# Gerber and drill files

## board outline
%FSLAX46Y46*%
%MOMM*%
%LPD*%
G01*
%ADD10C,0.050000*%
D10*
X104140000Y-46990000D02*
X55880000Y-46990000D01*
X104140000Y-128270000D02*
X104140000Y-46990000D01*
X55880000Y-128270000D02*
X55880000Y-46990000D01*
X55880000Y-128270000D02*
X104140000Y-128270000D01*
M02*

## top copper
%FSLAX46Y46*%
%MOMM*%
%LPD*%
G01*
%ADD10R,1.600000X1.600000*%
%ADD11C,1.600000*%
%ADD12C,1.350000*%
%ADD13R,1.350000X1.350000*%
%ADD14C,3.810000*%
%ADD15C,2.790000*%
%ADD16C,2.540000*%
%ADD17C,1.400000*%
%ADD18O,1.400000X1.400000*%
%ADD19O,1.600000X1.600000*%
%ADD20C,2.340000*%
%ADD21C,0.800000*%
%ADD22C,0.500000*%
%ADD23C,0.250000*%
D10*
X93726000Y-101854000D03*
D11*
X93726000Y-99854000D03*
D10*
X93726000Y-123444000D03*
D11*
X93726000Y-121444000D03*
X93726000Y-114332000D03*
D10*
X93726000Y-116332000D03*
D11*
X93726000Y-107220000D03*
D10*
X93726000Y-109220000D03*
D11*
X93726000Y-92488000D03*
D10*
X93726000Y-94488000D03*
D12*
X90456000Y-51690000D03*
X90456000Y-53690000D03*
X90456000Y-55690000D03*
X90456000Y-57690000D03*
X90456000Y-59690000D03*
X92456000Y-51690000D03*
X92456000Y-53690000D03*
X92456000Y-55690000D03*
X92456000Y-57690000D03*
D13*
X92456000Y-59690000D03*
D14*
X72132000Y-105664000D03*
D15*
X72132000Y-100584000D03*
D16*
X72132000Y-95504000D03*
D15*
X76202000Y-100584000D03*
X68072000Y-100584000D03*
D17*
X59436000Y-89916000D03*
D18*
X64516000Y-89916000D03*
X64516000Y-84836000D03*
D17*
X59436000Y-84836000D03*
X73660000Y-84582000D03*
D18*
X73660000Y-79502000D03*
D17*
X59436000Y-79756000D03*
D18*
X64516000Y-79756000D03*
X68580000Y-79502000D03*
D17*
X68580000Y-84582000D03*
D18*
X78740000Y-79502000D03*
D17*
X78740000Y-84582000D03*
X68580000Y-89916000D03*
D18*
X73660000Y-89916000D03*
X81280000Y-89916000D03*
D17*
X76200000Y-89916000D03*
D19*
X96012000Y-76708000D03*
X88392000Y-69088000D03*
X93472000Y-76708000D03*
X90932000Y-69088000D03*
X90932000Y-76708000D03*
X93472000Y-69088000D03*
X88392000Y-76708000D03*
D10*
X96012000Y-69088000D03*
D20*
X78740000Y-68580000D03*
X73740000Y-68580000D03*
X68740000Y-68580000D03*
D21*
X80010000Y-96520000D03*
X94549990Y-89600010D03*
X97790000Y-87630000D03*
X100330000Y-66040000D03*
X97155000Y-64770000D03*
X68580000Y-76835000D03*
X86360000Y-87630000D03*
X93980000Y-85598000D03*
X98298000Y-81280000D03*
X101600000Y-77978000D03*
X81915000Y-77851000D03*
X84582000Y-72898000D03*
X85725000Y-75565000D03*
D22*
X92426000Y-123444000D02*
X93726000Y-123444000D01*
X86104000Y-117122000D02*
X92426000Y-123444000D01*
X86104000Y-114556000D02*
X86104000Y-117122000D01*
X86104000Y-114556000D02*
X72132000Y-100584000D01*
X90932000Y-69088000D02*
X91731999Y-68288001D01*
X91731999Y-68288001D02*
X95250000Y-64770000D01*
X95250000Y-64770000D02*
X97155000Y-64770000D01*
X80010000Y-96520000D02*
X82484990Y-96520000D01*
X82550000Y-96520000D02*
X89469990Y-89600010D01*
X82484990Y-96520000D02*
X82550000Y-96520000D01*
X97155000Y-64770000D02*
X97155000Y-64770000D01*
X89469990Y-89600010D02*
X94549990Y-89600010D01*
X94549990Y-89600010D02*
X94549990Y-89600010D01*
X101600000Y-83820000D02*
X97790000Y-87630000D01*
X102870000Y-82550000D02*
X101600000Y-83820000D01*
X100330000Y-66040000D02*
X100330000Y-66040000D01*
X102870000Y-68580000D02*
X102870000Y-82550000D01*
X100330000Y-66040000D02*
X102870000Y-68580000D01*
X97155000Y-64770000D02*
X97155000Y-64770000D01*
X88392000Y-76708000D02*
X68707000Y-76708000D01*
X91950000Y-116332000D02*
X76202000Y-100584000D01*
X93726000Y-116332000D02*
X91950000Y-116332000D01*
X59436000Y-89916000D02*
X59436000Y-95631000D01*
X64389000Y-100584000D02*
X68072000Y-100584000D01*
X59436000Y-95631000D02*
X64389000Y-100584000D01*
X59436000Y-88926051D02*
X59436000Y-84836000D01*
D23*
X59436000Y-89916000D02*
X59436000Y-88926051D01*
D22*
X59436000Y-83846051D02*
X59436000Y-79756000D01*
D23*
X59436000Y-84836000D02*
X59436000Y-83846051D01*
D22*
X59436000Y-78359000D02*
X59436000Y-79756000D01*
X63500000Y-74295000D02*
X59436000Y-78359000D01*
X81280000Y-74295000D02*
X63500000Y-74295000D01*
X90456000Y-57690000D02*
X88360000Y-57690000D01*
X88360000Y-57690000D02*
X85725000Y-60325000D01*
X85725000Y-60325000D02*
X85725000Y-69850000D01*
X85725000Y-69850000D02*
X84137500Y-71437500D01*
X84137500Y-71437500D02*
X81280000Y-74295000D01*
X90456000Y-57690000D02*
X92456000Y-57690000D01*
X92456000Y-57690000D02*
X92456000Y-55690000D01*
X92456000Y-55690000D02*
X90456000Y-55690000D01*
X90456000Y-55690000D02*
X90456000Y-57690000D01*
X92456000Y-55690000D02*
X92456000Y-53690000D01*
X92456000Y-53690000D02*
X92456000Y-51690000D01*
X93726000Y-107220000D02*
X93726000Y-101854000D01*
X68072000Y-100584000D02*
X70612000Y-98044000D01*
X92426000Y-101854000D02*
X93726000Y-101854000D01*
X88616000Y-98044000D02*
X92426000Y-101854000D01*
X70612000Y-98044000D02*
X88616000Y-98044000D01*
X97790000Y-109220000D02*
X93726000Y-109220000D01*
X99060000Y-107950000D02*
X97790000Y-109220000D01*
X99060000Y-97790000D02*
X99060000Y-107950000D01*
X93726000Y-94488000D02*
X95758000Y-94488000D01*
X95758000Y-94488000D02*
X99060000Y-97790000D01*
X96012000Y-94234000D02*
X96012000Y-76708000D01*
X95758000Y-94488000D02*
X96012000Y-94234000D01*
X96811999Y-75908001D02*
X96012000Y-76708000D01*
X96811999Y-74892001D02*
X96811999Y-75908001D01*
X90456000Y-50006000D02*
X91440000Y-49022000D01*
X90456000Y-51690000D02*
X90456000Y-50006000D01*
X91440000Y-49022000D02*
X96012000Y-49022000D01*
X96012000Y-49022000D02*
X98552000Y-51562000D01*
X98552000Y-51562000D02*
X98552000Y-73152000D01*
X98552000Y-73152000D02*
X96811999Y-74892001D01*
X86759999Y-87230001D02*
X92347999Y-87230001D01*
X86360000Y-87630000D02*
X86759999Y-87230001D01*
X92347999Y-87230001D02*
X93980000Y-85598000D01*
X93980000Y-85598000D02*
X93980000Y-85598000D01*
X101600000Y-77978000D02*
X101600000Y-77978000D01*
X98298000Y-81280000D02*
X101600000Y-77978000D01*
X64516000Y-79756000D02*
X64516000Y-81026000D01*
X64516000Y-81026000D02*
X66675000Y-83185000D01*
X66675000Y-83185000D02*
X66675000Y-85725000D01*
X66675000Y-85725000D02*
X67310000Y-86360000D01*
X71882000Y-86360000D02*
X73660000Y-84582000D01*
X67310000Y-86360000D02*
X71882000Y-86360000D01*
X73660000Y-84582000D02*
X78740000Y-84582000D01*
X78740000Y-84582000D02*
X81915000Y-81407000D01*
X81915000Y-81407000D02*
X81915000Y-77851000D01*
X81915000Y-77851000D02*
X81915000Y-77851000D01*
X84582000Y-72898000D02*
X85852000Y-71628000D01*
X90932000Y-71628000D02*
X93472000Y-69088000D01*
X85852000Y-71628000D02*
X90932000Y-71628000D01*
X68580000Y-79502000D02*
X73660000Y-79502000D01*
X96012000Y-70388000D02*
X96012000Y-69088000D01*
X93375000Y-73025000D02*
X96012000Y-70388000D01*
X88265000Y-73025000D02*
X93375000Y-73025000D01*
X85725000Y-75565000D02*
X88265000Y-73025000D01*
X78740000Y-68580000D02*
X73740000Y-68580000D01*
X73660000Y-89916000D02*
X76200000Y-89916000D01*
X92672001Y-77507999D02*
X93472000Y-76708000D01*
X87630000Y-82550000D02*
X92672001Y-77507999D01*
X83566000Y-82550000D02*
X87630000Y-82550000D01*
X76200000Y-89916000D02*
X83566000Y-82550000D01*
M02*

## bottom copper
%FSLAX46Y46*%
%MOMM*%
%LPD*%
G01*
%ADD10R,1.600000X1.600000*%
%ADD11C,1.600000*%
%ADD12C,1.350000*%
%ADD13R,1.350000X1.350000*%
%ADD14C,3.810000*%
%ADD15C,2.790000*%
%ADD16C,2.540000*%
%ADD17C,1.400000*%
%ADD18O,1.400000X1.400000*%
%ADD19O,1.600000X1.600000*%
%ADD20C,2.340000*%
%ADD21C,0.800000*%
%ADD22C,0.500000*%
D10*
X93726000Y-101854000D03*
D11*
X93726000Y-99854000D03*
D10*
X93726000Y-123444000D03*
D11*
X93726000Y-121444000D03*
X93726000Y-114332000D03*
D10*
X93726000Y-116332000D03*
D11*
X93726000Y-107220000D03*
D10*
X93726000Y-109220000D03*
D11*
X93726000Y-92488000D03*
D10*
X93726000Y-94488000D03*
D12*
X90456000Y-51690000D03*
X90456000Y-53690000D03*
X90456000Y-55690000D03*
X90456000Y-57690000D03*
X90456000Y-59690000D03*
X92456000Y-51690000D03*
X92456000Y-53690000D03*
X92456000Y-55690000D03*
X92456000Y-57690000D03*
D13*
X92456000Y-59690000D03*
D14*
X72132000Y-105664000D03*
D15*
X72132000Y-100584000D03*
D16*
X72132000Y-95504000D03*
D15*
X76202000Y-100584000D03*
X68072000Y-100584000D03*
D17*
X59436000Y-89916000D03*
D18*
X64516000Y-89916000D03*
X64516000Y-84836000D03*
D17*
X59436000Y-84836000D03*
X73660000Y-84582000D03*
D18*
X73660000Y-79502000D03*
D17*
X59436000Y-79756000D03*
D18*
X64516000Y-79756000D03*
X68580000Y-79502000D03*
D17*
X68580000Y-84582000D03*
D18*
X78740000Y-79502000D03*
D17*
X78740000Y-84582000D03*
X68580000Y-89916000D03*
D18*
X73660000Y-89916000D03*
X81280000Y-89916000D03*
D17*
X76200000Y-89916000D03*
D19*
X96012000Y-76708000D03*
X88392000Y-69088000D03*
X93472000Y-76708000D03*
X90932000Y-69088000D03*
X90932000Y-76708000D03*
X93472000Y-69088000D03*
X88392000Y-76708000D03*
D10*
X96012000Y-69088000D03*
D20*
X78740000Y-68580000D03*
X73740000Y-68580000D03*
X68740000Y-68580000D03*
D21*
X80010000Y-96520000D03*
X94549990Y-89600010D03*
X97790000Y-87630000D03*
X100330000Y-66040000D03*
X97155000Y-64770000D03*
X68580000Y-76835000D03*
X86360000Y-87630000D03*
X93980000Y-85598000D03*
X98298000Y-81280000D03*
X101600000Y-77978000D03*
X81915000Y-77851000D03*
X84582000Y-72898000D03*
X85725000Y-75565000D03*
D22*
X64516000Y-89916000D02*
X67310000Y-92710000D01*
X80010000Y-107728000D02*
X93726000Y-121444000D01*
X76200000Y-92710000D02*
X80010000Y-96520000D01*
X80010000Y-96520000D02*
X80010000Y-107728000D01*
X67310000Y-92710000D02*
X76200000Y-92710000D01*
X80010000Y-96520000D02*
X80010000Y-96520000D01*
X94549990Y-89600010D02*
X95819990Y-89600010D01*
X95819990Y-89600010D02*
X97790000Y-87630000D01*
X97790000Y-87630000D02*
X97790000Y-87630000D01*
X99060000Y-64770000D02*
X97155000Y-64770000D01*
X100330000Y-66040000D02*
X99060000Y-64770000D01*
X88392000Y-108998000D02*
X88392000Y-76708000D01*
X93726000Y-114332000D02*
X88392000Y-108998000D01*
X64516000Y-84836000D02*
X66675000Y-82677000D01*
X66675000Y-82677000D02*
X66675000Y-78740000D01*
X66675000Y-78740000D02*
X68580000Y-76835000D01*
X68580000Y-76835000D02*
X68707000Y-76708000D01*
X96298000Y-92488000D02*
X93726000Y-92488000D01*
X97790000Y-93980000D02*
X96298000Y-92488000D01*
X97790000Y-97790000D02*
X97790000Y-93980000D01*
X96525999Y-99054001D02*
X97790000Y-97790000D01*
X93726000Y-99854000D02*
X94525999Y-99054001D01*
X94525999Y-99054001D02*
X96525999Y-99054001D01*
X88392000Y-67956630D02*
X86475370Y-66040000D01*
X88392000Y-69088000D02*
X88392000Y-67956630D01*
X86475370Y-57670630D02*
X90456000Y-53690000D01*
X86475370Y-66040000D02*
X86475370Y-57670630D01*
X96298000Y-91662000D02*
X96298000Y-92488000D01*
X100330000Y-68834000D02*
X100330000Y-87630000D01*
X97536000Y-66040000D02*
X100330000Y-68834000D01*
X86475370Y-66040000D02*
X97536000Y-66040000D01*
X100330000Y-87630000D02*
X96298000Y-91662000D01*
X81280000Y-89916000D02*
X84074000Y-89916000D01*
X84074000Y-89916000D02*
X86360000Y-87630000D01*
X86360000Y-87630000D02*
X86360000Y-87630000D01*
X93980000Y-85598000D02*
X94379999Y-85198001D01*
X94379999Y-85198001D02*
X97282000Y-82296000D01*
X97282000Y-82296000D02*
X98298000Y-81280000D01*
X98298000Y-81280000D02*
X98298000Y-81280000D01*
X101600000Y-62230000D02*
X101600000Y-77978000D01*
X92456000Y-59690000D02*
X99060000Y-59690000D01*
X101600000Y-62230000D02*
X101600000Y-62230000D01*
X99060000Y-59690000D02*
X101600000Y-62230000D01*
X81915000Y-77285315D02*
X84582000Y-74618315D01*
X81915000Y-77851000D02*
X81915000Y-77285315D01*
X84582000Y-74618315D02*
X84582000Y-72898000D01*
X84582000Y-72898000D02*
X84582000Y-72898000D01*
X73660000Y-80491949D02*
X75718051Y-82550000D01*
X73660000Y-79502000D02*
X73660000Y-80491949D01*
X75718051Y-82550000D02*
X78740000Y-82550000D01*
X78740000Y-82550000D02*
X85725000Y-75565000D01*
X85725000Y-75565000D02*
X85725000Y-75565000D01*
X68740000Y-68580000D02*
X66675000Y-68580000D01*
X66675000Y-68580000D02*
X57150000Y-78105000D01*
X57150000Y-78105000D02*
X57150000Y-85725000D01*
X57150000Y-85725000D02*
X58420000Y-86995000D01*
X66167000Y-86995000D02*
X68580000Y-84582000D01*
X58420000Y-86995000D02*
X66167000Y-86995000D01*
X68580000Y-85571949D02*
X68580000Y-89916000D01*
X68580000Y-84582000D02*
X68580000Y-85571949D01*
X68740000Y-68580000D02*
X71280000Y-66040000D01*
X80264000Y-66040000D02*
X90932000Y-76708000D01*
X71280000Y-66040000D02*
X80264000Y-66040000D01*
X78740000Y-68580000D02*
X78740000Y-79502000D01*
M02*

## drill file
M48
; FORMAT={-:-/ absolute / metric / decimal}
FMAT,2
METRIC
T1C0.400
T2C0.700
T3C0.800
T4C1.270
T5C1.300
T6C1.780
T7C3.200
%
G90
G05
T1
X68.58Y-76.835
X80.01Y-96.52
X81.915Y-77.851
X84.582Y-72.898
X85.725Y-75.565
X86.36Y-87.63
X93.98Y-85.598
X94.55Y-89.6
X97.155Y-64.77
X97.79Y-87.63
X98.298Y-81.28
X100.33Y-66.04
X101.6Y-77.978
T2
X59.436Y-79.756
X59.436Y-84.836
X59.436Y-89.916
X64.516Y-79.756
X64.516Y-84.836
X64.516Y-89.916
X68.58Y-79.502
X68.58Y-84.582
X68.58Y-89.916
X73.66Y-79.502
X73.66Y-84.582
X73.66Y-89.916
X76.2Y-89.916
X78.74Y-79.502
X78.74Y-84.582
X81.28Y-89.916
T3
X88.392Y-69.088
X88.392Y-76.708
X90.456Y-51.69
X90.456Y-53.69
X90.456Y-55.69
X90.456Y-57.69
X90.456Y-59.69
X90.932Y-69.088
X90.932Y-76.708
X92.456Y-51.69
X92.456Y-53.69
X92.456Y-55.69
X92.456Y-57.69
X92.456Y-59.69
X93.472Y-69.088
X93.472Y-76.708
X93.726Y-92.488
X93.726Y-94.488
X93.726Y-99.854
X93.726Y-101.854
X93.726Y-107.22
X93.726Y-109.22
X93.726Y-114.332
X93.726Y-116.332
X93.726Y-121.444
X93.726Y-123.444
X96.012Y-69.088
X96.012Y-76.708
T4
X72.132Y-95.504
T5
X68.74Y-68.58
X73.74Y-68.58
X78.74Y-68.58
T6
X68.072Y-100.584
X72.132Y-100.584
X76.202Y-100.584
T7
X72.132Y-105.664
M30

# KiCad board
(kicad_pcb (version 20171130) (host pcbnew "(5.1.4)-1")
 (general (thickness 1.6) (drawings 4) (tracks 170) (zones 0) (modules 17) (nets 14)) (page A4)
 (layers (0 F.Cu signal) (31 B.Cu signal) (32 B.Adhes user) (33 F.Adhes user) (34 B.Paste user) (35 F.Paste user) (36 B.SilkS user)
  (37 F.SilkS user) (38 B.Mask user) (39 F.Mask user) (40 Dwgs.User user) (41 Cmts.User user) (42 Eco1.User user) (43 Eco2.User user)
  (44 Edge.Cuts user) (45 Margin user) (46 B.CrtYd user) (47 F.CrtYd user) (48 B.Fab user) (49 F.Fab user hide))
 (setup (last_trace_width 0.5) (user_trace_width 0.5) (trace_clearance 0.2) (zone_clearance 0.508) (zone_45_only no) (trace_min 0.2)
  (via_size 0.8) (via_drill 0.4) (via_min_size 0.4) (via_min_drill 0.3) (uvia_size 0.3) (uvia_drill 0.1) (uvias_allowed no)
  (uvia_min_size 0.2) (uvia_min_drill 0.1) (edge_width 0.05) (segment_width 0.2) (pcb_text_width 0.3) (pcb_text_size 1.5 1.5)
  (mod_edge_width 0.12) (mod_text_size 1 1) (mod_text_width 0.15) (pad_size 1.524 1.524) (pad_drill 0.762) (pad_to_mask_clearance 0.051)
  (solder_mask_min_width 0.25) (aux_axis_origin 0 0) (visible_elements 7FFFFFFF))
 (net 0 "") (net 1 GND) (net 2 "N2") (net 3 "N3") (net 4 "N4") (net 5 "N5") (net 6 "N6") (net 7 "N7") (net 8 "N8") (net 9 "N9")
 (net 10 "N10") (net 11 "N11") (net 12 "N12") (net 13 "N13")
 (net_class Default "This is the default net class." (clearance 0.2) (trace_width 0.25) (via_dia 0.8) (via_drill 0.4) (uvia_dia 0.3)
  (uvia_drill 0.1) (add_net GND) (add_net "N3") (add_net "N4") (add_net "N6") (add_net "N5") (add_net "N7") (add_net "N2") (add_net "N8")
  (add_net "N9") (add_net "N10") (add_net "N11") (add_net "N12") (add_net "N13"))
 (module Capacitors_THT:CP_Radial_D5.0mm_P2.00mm (layer F.Cu) (at 93.726 101.854 90)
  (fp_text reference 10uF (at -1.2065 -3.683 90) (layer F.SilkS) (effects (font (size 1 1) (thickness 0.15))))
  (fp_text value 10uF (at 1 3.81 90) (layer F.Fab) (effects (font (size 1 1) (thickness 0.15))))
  (pad 1 thru_hole rect (at 0 0 90) (size 1.6 1.6) (drill 0.8) (layers *.Cu *.Mask) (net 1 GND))
  (pad 2 thru_hole circle (at 2 0 90) (size 1.6 1.6) (drill 0.8) (layers *.Cu *.Mask) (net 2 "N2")))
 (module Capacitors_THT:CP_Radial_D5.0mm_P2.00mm (layer F.Cu) (at 93.726 123.444 90)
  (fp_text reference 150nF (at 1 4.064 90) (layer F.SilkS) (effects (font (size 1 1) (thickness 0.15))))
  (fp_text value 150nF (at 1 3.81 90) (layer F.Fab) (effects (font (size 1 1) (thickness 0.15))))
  (pad 1 thru_hole rect (at 0 0 90) (size 1.6 1.6) (drill 0.8) (layers *.Cu *.Mask) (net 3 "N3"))
  (pad 2 thru_hole circle (at 2 0 90) (size 1.6 1.6) (drill 0.8) (layers *.Cu *.Mask) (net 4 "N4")))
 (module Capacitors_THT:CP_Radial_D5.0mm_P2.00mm (layer F.Cu) (at 93.726 116.332 90)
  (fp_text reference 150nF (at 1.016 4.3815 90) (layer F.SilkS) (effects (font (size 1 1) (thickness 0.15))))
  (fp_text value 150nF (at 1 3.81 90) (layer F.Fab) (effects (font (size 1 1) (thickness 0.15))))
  (pad 2 thru_hole circle (at 2 0 90) (size 1.6 1.6) (drill 0.8) (layers *.Cu *.Mask) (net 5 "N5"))
  (pad 1 thru_hole rect (at 0 0 90) (size 1.6 1.6) (drill 0.8) (layers *.Cu *.Mask) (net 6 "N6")))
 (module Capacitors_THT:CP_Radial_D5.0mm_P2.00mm (layer F.Cu) (at 93.726 109.22 90)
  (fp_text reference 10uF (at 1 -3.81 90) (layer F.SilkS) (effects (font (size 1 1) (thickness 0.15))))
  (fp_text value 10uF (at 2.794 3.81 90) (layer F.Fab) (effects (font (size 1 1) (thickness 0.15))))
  (pad 2 thru_hole circle (at 2 0 90) (size 1.6 1.6) (drill 0.8) (layers *.Cu *.Mask) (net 1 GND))
  (pad 1 thru_hole rect (at 0 0 90) (size 1.6 1.6) (drill 0.8) (layers *.Cu *.Mask) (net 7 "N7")))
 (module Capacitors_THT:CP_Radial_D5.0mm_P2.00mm (layer F.Cu) (at 93.726 94.488 90)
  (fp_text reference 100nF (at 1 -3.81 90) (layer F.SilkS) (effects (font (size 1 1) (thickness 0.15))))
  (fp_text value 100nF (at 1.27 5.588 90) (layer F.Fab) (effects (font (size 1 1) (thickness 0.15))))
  (pad 2 thru_hole circle (at 2 0 90) (size 1.6 1.6) (drill 0.8) (layers *.Cu *.Mask) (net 2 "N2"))
  (pad 1 thru_hole rect (at 0 0 90) (size 1.6 1.6) (drill 0.8) (layers *.Cu *.Mask) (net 7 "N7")))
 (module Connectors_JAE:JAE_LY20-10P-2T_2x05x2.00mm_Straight (layer F.Cu) (at 92.456 59.69 90)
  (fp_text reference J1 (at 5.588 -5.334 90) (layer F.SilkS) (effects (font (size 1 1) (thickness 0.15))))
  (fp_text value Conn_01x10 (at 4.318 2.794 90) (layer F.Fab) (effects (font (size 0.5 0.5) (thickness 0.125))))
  (pad 10 thru_hole circle (at 8 -2 90) (size 1.35 1.35) (drill 0.8) (layers *.Cu *.Mask) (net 7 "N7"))
  (pad 9 thru_hole circle (at 6 -2 90) (size 1.35 1.35) (drill 0.8) (layers *.Cu *.Mask) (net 2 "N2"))
  (pad 8 thru_hole circle (at 4 -2 90) (size 1.35 1.35) (drill 0.8) (layers *.Cu *.Mask) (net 1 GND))
  (pad 7 thru_hole circle (at 2 -2 90) (size 1.35 1.35) (drill 0.8) (layers *.Cu *.Mask) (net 1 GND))
  (pad 6 thru_hole circle (at 0 -2 90) (size 1.35 1.35) (drill 0.8) (layers *.Cu *.Mask))
  (pad 5 thru_hole circle (at 8 0 90) (size 1.35 1.35) (drill 0.8) (layers *.Cu *.Mask) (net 1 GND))
  (pad 4 thru_hole circle (at 6 0 90) (size 1.35 1.35) (drill 0.8) (layers *.Cu *.Mask) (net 1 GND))
  (pad 3 thru_hole circle (at 4 0 90) (size 1.35 1.35) (drill 0.8) (layers *.Cu *.Mask) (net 1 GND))
  (pad 2 thru_hole circle (at 2 0 90) (size 1.35 1.35) (drill 0.8) (layers *.Cu *.Mask) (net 1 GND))
  (pad 1 thru_hole rect (at 0 0 90) (size 1.35 1.35) (drill 0.8) (layers *.Cu *.Mask) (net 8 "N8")))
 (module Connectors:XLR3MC (layer F.Cu) (at 68.072 100.584)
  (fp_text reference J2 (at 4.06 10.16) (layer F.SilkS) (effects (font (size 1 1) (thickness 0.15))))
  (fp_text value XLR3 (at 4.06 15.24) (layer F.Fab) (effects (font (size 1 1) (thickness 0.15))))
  (pad "" thru_hole circle (at 4.06 5.08) (size 3.81 3.81) (drill 3.2) (layers *.Cu *.Mask))
  (pad 3 thru_hole circle (at 4.06 0) (size 2.79 2.79) (drill 1.78) (layers *.Cu *.Mask) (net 3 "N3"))
  (pad 4 thru_hole circle (at 4.06 -5.08) (size 2.54 2.54) (drill 1.27) (layers *.Cu *.Mask))
  (pad 2 thru_hole circle (at 8.13 0) (size 2.79 2.79) (drill 1.78) (layers *.Cu *.Mask) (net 6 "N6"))
  (pad 1 thru_hole circle (at 0 0) (size 2.79 2.79) (drill 1.78) (layers *.Cu *.Mask) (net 1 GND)))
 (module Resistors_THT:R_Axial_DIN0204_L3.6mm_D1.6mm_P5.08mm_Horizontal (layer F.Cu) (at 59.436 89.916)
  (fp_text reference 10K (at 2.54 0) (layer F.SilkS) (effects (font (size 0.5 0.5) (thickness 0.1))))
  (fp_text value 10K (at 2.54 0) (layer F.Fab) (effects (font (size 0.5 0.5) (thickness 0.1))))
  (pad 1 thru_hole circle (at 0 0) (size 1.4 1.4) (drill 0.7) (layers *.Cu *.Mask) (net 1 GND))
  (pad 2 thru_hole oval (at 5.08 0) (size 1.4 1.4) (drill 0.7) (layers *.Cu *.Mask) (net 4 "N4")))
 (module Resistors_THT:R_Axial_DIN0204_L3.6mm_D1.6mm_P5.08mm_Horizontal (layer F.Cu) (at 59.436 84.836)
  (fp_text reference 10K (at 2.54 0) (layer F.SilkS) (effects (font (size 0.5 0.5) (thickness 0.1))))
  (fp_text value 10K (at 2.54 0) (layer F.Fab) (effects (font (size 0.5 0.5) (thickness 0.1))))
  (pad 2 thru_hole oval (at 5.08 0) (size 1.4 1.4) (drill 0.7) (layers *.Cu *.Mask) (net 5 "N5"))
  (pad 1 thru_hole circle (at 0 0) (size 1.4 1.4) (drill 0.7) (layers *.Cu *.Mask) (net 1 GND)))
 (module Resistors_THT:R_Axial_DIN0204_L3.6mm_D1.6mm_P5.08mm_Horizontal (layer F.Cu) (at 73.66 84.582 90)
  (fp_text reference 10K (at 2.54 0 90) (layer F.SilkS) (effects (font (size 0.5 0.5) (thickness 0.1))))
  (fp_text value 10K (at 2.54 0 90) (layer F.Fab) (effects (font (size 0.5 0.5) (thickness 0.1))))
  (pad 1 thru_hole circle (at 0 0 90) (size 1.4 1.4) (drill 0.7) (layers *.Cu *.Mask) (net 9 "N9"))
  (pad 2 thru_hole oval (at 5.08 0 90) (size 1.4 1.4) (drill 0.7) (layers *.Cu *.Mask) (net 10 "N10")))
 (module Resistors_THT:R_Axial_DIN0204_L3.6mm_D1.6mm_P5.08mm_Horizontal (layer F.Cu) (at 59.436 79.756)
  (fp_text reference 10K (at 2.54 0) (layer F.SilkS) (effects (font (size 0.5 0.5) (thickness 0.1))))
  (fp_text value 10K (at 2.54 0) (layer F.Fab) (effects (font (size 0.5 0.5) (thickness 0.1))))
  (pad 1 thru_hole circle (at 0 0) (size 1.4 1.4) (drill 0.7) (layers *.Cu *.Mask) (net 1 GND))
  (pad 2 thru_hole oval (at 5.08 0) (size 1.4 1.4) (drill 0.7) (layers *.Cu *.Mask) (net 9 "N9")))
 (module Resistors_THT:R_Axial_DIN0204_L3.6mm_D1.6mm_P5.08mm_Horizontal (layer F.Cu) (at 68.58 84.582 90)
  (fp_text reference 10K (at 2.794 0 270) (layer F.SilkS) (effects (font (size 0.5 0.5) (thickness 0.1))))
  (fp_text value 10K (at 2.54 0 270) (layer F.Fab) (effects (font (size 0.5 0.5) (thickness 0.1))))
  (pad 2 thru_hole oval (at 5.08 0 90) (size 1.4 1.4) (drill 0.7) (layers *.Cu *.Mask) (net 10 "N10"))
  (pad 1 thru_hole circle (at 0 0 90) (size 1.4 1.4) (drill 0.7) (layers *.Cu *.Mask) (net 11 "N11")))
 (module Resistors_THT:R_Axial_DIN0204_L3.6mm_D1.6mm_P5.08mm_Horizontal (layer F.Cu) (at 78.74 84.582 90)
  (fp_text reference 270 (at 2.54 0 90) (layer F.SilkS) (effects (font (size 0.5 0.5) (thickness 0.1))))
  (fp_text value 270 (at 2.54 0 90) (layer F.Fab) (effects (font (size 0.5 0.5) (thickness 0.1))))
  (pad 2 thru_hole oval (at 5.08 0 90) (size 1.4 1.4) (drill 0.7) (layers *.Cu *.Mask) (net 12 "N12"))
  (pad 1 thru_hole circle (at 0 0 90) (size 1.4 1.4) (drill 0.7) (layers *.Cu *.Mask) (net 9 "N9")))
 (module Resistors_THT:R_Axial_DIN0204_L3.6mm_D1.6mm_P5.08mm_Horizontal (layer F.Cu) (at 68.58 89.916)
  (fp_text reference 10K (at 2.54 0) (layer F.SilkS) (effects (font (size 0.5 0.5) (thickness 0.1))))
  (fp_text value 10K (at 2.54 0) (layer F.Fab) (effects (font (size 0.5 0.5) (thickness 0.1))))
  (pad 1 thru_hole circle (at 0 0) (size 1.4 1.4) (drill 0.7) (layers *.Cu *.Mask) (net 11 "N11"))
  (pad 2 thru_hole oval (at 5.08 0) (size 1.4 1.4) (drill 0.7) (layers *.Cu *.Mask) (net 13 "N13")))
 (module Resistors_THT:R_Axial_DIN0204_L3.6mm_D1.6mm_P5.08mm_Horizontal (layer F.Cu) (at 76.2 89.916)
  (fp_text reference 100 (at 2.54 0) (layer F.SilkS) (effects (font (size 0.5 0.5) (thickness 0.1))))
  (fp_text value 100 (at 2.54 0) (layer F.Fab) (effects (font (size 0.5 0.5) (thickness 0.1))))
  (pad 2 thru_hole oval (at 5.08 0) (size 1.4 1.4) (drill 0.7) (layers *.Cu *.Mask) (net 8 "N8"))
  (pad 1 thru_hole circle (at 0 0) (size 1.4 1.4) (drill 0.7) (layers *.Cu *.Mask) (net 13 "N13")))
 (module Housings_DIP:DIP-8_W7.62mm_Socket (layer F.Cu) (at 96.012 69.088 270)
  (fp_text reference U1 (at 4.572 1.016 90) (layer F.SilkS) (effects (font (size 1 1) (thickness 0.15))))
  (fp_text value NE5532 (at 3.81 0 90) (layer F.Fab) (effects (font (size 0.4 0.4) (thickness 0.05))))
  (pad 8 thru_hole oval (at 7.62 0 270) (size 1.6 1.6) (drill 0.8) (layers *.Cu *.Mask) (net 7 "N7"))
  (pad 4 thru_hole oval (at 0 7.62 270) (size 1.6 1.6) (drill 0.8) (layers *.Cu *.Mask) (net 2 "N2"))
  (pad 7 thru_hole oval (at 7.62 2.54 270) (size 1.6 1.6) (drill 0.8) (layers *.Cu *.Mask) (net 13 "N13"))
  (pad 3 thru_hole oval (at 0 5.08 270) (size 1.6 1.6) (drill 0.8) (layers *.Cu *.Mask) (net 4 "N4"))
  (pad 6 thru_hole oval (at 7.62 5.08 270) (size 1.6 1.6) (drill 0.8) (layers *.Cu *.Mask) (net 11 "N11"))
  (pad 2 thru_hole oval (at 0 2.54 270) (size 1.6 1.6) (drill 0.8) (layers *.Cu *.Mask) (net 9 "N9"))
  (pad 5 thru_hole oval (at 7.62 7.62 270) (size 1.6 1.6) (drill 0.8) (layers *.Cu *.Mask) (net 5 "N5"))
  (pad 1 thru_hole rect (at 0 0 270) (size 1.6 1.6) (drill 0.8) (layers *.Cu *.Mask) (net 10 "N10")))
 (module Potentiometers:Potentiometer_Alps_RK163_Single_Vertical (layer F.Cu) (at 78.74 68.58 90)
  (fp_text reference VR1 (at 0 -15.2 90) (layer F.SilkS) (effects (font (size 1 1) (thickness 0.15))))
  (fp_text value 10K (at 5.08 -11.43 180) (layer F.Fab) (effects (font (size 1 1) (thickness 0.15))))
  (pad 1 thru_hole circle (at 0 0 90) (size 2.34 2.34) (drill 1.3) (layers *.Cu *.Mask) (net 12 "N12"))
  (pad 2 thru_hole circle (at 0 -5 90) (size 2.34 2.34) (drill 1.3) (layers *.Cu *.Mask) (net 12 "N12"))
  (pad 3 thru_hole circle (at 0 -10 90) (size 2.34 2.34) (drill 1.3) (layers *.Cu *.Mask) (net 11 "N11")))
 (gr_line (start 104.14 46.99) (end 55.88 46.99) (layer Edge.Cuts) (width 0.05))
 (gr_line (start 104.14 128.27) (end 104.14 46.99) (layer Edge.Cuts) (width 0.05))
 (gr_line (start 55.88 128.27) (end 55.88 46.99) (layer Edge.Cuts) (width 0.05))
 (gr_line (start 55.88 128.27) (end 104.14 128.27) (layer Edge.Cuts) (width 0.05))
 (segment (start 92.426 123.444) (end 93.726 123.444) (width 0.5) (layer F.Cu) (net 3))
 (segment (start 86.104 117.122) (end 92.426 123.444) (width 0.5) (layer F.Cu) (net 3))
 (segment (start 86.104 114.556) (end 86.104 117.122) (width 0.5) (layer F.Cu) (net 3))
 (segment (start 86.104 114.556) (end 72.132 100.584) (width 0.5) (layer F.Cu) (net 3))
 (segment (start 64.516 89.916) (end 67.31 92.71) (width 0.5) (layer B.Cu) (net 4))
 (segment (start 80.01 107.728) (end 93.726 121.444) (width 0.5) (layer B.Cu) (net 4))
 (segment (start 76.2 92.71) (end 80.01 96.52) (width 0.5) (layer B.Cu) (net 4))
 (segment (start 80.01 96.52) (end 80.01 107.728) (width 0.5) (layer B.Cu) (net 4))
 (segment (start 67.31 92.71) (end 76.2 92.71) (width 0.5) (layer B.Cu) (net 4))
 (segment (start 90.932 69.088) (end 91.731999 68.288001) (width 0.5) (layer F.Cu) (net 4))
 (segment (start 91.731999 68.288001) (end 95.25 64.77) (width 0.5) (layer F.Cu) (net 4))
 (segment (start 95.25 64.77) (end 97.155 64.77) (width 0.5) (layer F.Cu) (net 4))
 (segment (start 80.01 96.52) (end 80.01 96.52) (width 0.5) (layer B.Cu) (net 4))
 (via (at 80.01 96.52) (size 0.8) (drill 0.4) (layers F.Cu B.Cu) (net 4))
 (segment (start 80.01 96.52) (end 82.48499 96.52) (width 0.5) (layer F.Cu) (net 4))
 (segment (start 82.55 96.52) (end 89.46999 89.60001) (width 0.5) (layer F.Cu) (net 4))
 (segment (start 82.48499 96.52) (end 82.55 96.52) (width 0.5) (layer F.Cu) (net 4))
 (segment (start 97.155 64.77) (end 97.155 64.77) (width 0.5) (layer F.Cu) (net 4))
 (segment (start 89.46999 89.60001) (end 94.54999 89.60001) (width 0.5) (layer F.Cu) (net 4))
 (segment (start 94.54999 89.60001) (end 94.54999 89.60001) (width 0.5) (layer F.Cu) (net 4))
 (via (at 94.54999 89.60001) (size 0.8) (drill 0.4) (layers F.Cu B.Cu) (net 4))
 (segment (start 94.54999 89.60001) (end 95.81999 89.60001) (width 0.5) (layer B.Cu) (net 4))
 (segment (start 95.81999 89.60001) (end 97.79 87.63) (width 0.5) (layer B.Cu) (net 4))
 (segment (start 97.79 87.63) (end 97.79 87.63) (width 0.5) (layer B.Cu) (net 4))
 (via (at 97.79 87.63) (size 0.8) (drill 0.4) (layers F.Cu B.Cu) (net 4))
 (segment (start 101.6 83.82) (end 97.79 87.63) (width 0.5) (layer F.Cu) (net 4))
 (segment (start 102.87 82.55) (end 101.6 83.82) (width 0.5) (layer F.Cu) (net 4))
 (segment (start 100.33 66.04) (end 100.33 66.04) (width 0.5) (layer F.Cu) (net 4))
 (segment (start 102.87 68.58) (end 102.87 82.55) (width 0.5) (layer F.Cu) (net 4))
 (segment (start 100.33 66.04) (end 102.87 68.58) (width 0.5) (layer F.Cu) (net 4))
 (via (at 100.33 66.04) (size 0.8) (drill 0.4) (layers F.Cu B.Cu) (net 4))
 (segment (start 97.155 64.77) (end 97.155 64.77) (width 0.5) (layer F.Cu) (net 4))
 (via (at 97.155 64.77) (size 0.8) (drill 0.4) (layers F.Cu B.Cu) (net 4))
 (segment (start 99.06 64.77) (end 97.155 64.77) (width 0.5) (layer B.Cu) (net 4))
 (segment (start 100.33 66.04) (end 99.06 64.77) (width 0.5) (layer B.Cu) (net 4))
 (segment (start 88.392 108.998) (end 88.392 76.708) (width 0.5) (layer B.Cu) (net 5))
 (segment (start 93.726 114.332) (end 88.392 108.998) (width 0.5) (layer B.Cu) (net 5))
 (segment (start 64.516 84.836) (end 66.675 82.677) (width 0.5) (layer B.Cu) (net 5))
 (segment (start 66.675 82.677) (end 66.675 78.74) (width 0.5) (layer B.Cu) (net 5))
 (segment (start 66.675 78.74) (end 68.58 76.835) (width 0.5) (layer B.Cu) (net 5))
 (segment (start 88.392 76.708) (end 68.707 76.708) (width 0.5) (layer F.Cu) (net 5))
 (segment (start 68.58 76.835) (end 68.707 76.708) (width 0.5) (layer B.Cu) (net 5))
 (via (at 68.58 76.835) (size 0.8) (drill 0.4) (layers F.Cu B.Cu) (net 5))
 (segment (start 91.95 116.332) (end 76.202 100.584) (width 0.5) (layer F.Cu) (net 6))
 (segment (start 93.726 116.332) (end 91.95 116.332) (width 0.5) (layer F.Cu) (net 6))
 (segment (start 59.436 89.916) (end 59.436 95.631) (width 0.5) (layer F.Cu) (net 1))
 (segment (start 64.389 100.584) (end 68.072 100.584) (width 0.5) (layer F.Cu) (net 1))
 (segment (start 59.436 95.631) (end 64.389 100.584) (width 0.5) (layer F.Cu) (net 1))
 (segment (start 59.436 88.926051) (end 59.436 84.836) (width 0.5) (layer F.Cu) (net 1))
 (segment (start 59.436 89.916) (end 59.436 88.926051) (width 0.25) (layer F.Cu) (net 1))
 (segment (start 59.436 83.846051) (end 59.436 79.756) (width 0.5) (layer F.Cu) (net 1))
 (segment (start 59.436 84.836) (end 59.436 83.846051) (width 0.25) (layer F.Cu) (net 1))
 (segment (start 59.436 78.359) (end 59.436 79.756) (width 0.5) (layer F.Cu) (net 1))
 (segment (start 63.5 74.295) (end 59.436 78.359) (width 0.5) (layer F.Cu) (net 1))
 (segment (start 81.28 74.295) (end 63.5 74.295) (width 0.5) (layer F.Cu) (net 1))
 (segment (start 90.456 57.69) (end 88.36 57.69) (width 0.5) (layer F.Cu) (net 1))
 (segment (start 88.36 57.69) (end 85.725 60.325) (width 0.5) (layer F.Cu) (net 1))
 (segment (start 85.725 60.325) (end 85.725 69.85) (width 0.5) (layer F.Cu) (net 1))
 (segment (start 85.725 69.85) (end 84.1375 71.4375) (width 0.5) (layer F.Cu) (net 1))
 (segment (start 84.1375 71.4375) (end 81.28 74.295) (width 0.5) (layer F.Cu) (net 1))
 (segment (start 90.456 57.69) (end 92.456 57.69) (width 0.5) (layer F.Cu) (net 1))
 (segment (start 92.456 57.69) (end 92.456 55.69) (width 0.5) (layer F.Cu) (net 1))
 (segment (start 92.456 55.69) (end 90.456 55.69) (width 0.5) (layer F.Cu) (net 1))
 (segment (start 90.456 55.69) (end 90.456 57.69) (width 0.5) (layer F.Cu) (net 1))
 (segment (start 92.456 55.69) (end 92.456 53.69) (width 0.5) (layer F.Cu) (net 1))
 (segment (start 92.456 53.69) (end 92.456 51.69) (width 0.5) (layer F.Cu) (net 1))
 (segment (start 93.726 107.22) (end 93.726 101.854) (width 0.5) (layer F.Cu) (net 1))
 (segment (start 68.072 100.584) (end 70.612 98.044) (width 0.5) (layer F.Cu) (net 1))
 (segment (start 92.426 101.854) (end 93.726 101.854) (width 0.5) (layer F.Cu) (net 1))
 (segment (start 88.616 98.044) (end 92.426 101.854) (width 0.5) (layer F.Cu) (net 1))
 (segment (start 70.612 98.044) (end 88.616 98.044) (width 0.5) (layer F.Cu) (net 1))
 (segment (start 97.79 109.22) (end 93.726 109.22) (width 0.5) (layer F.Cu) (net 7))
 (segment (start 99.06 107.95) (end 97.79 109.22) (width 0.5) (layer F.Cu) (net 7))
 (segment (start 99.06 97.79) (end 99.06 107.95) (width 0.5) (layer F.Cu) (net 7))
 (segment (start 93.726 94.488) (end 95.758 94.488) (width 0.5) (layer F.Cu) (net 7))
 (segment (start 95.758 94.488) (end 99.06 97.79) (width 0.5) (layer F.Cu) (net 7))
 (segment (start 96.012 94.234) (end 96.012 76.708) (width 0.5) (layer F.Cu) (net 7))
 (segment (start 95.758 94.488) (end 96.012 94.234) (width 0.5) (layer F.Cu) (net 7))
 (segment (start 96.811999 75.908001) (end 96.012 76.708) (width 0.5) (layer F.Cu) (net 7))
 (segment (start 96.811999 74.892001) (end 96.811999 75.908001) (width 0.5) (layer F.Cu) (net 7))
 (segment (start 90.456 50.006) (end 91.44 49.022) (width 0.5) (layer F.Cu) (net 7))
 (segment (start 90.456 51.69) (end 90.456 50.006) (width 0.5) (layer F.Cu) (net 7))
 (segment (start 91.44 49.022) (end 96.012 49.022) (width 0.5) (layer F.Cu) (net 7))
 (segment (start 96.012 49.022) (end 98.552 51.562) (width 0.5) (layer F.Cu) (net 7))
 (segment (start 98.552 51.562) (end 98.552 73.152) (width 0.5) (layer F.Cu) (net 7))
 (segment (start 98.552 73.152) (end 96.811999 74.892001) (width 0.5) (layer F.Cu) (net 7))
 (segment (start 96.298 92.488) (end 93.726 92.488) (width 0.5) (layer B.Cu) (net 2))
 (segment (start 97.79 93.98) (end 96.298 92.488) (width 0.5) (layer B.Cu) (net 2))
 (segment (start 97.79 97.79) (end 97.79 93.98) (width 0.5) (layer B.Cu) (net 2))
 (segment (start 96.525999 99.054001) (end 97.79 97.79) (width 0.5) (layer B.Cu) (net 2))
 (segment (start 93.726 99.854) (end 94.525999 99.054001) (width 0.5) (layer B.Cu) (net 2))
 (segment (start 94.525999 99.054001) (end 96.525999 99.054001) (width 0.5) (layer B.Cu) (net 2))
 (segment (start 88.392 67.95663) (end 86.47537 66.04) (width 0.5) (layer B.Cu) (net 2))
 (segment (start 88.392 69.088) (end 88.392 67.95663) (width 0.5) (layer B.Cu) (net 2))
 (segment (start 86.47537 57.67063) (end 90.456 53.69) (width 0.5) (layer B.Cu) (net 2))
 (segment (start 86.47537 66.04) (end 86.47537 57.67063) (width 0.5) (layer B.Cu) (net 2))
 (segment (start 96.298 91.662) (end 96.298 92.488) (width 0.5) (layer B.Cu) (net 2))
 (segment (start 100.33 68.834) (end 100.33 87.63) (width 0.5) (layer B.Cu) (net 2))
 (segment (start 97.536 66.04) (end 100.33 68.834) (width 0.5) (layer B.Cu) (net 2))
 (segment (start 86.47537 66.04) (end 97.536 66.04) (width 0.5) (layer B.Cu) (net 2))
 (segment (start 100.33 87.63) (end 96.298 91.662) (width 0.5) (layer B.Cu) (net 2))
 (segment (start 81.28 89.916) (end 84.074 89.916) (width 0.5) (layer B.Cu) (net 8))
 (segment (start 84.074 89.916) (end 86.36 87.63) (width 0.5) (layer B.Cu) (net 8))
 (segment (start 86.36 87.63) (end 86.36 87.63) (width 0.5) (layer B.Cu) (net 8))
 (via (at 86.36 87.63) (size 0.8) (drill 0.4) (layers F.Cu B.Cu) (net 8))
 (segment (start 86.759999 87.230001) (end 92.347999 87.230001) (width 0.5) (layer F.Cu) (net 8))
 (segment (start 86.36 87.63) (end 86.759999 87.230001) (width 0.5) (layer F.Cu) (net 8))
 (segment (start 92.347999 87.230001) (end 93.98 85.598) (width 0.5) (layer F.Cu) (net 8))
 (segment (start 93.98 85.598) (end 93.98 85.598) (width 0.5) (layer F.Cu) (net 8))
 (via (at 93.98 85.598) (size 0.8) (drill 0.4) (layers F.Cu B.Cu) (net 8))
 (segment (start 93.98 85.598) (end 94.379999 85.198001) (width 0.5) (layer B.Cu) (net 8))
 (segment (start 94.379999 85.198001) (end 97.282 82.296) (width 0.5) (layer B.Cu) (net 8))
 (segment (start 97.282 82.296) (end 98.298 81.28) (width 0.5) (layer B.Cu) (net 8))
 (segment (start 98.298 81.28) (end 98.298 81.28) (width 0.5) (layer B.Cu) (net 8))
 (via (at 98.298 81.28) (size 0.8) (drill 0.4) (layers F.Cu B.Cu) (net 8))
 (segment (start 101.6 62.23) (end 101.6 77.978) (width 0.5) (layer B.Cu) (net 8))
 (segment (start 92.456 59.69) (end 99.06 59.69) (width 0.5) (layer B.Cu) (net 8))
 (segment (start 101.6 77.978) (end 101.6 77.978) (width 0.5) (layer F.Cu) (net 8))
 (segment (start 98.298 81.28) (end 101.6 77.978) (width 0.5) (layer F.Cu) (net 8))
 (via (at 101.6 77.978) (size 0.8) (drill 0.4) (layers F.Cu B.Cu) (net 8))
 (segment (start 101.6 62.23) (end 101.6 62.23) (width 0.5) (layer B.Cu) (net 8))
 (segment (start 99.06 59.69) (end 101.6 62.23) (width 0.5) (layer B.Cu) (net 8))
 (segment (start 64.516 79.756) (end 64.516 81.026) (width 0.5) (layer F.Cu) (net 9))
 (segment (start 64.516 81.026) (end 66.675 83.185) (width 0.5) (layer F.Cu) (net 9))
 (segment (start 66.675 83.185) (end 66.675 85.725) (width 0.5) (layer F.Cu) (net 9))
 (segment (start 66.675 85.725) (end 67.31 86.36) (width 0.5) (layer F.Cu) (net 9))
 (segment (start 71.882 86.36) (end 73.66 84.582) (width 0.5) (layer F.Cu) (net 9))
 (segment (start 67.31 86.36) (end 71.882 86.36) (width 0.5) (layer F.Cu) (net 9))
 (segment (start 73.66 84.582) (end 78.74 84.582) (width 0.5) (layer F.Cu) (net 9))
 (segment (start 78.74 84.582) (end 81.915 81.407) (width 0.5) (layer F.Cu) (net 9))
 (segment (start 81.915 81.407) (end 81.915 77.851) (width 0.5) (layer F.Cu) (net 9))
 (segment (start 81.915 77.851) (end 81.915 77.851) (width 0.5) (layer F.Cu) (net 9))
 (via (at 81.915 77.851) (size 0.8) (drill 0.4) (layers F.Cu B.Cu) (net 9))
 (segment (start 81.915 77.285315) (end 84.582 74.618315) (width 0.5) (layer B.Cu) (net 9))
 (segment (start 81.915 77.851) (end 81.915 77.285315) (width 0.5) (layer B.Cu) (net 9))
 (segment (start 84.582 74.618315) (end 84.582 72.898) (width 0.5) (layer B.Cu) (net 9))
 (segment (start 84.582 72.898) (end 84.582 72.898) (width 0.5) (layer B.Cu) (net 9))
 (via (at 84.582 72.898) (size 0.8) (drill 0.4) (layers F.Cu B.Cu) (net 9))
 (segment (start 84.582 72.898) (end 85.852 71.628) (width 0.5) (layer F.Cu) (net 9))
 (segment (start 90.932 71.628) (end 93.472 69.088) (width 0.5) (layer F.Cu) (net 9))
 (segment (start 85.852 71.628) (end 90.932 71.628) (width 0.5) (layer F.Cu) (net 9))
 (segment (start 68.58 79.502) (end 73.66 79.502) (width 0.5) (layer F.Cu) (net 10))
 (segment (start 73.66 80.491949) (end 75.718051 82.55) (width 0.5) (layer B.Cu) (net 10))
 (segment (start 73.66 79.502) (end 73.66 80.491949) (width 0.5) (layer B.Cu) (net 10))
 (segment (start 75.718051 82.55) (end 78.74 82.55) (width 0.5) (layer B.Cu) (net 10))
 (segment (start 78.74 82.55) (end 85.725 75.565) (width 0.5) (layer B.Cu) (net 10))
 (segment (start 85.725 75.565) (end 85.725 75.565) (width 0.5) (layer B.Cu) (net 10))
 (via (at 85.725 75.565) (size 0.8) (drill 0.4) (layers F.Cu B.Cu) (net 10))
 (segment (start 96.012 70.388) (end 96.012 69.088) (width 0.5) (layer F.Cu) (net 10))
 (segment (start 93.375 73.025) (end 96.012 70.388) (width 0.5) (layer F.Cu) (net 10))
 (segment (start 88.265 73.025) (end 93.375 73.025) (width 0.5) (layer F.Cu) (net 10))
 (segment (start 85.725 75.565) (end 88.265 73.025) (width 0.5) (layer F.Cu) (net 10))
 (segment (start 68.74 68.58) (end 66.675 68.58) (width 0.5) (layer B.Cu) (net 11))
 (segment (start 66.675 68.58) (end 57.15 78.105) (width 0.5) (layer B.Cu) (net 11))
 (segment (start 57.15 78.105) (end 57.15 85.725) (width 0.5) (layer B.Cu) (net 11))
 (segment (start 57.15 85.725) (end 58.42 86.995) (width 0.5) (layer B.Cu) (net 11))
 (segment (start 66.167 86.995) (end 68.58 84.582) (width 0.5) (layer B.Cu) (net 11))
 (segment (start 58.42 86.995) (end 66.167 86.995) (width 0.5) (layer B.Cu) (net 11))
 (segment (start 68.58 85.571949) (end 68.58 89.916) (width 0.5) (layer B.Cu) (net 11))
 (segment (start 68.58 84.582) (end 68.58 85.571949) (width 0.5) (layer B.Cu) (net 11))
 (segment (start 68.74 68.58) (end 71.28 66.04) (width 0.5) (layer B.Cu) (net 11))
 (segment (start 80.264 66.04) (end 90.932 76.708) (width 0.5) (layer B.Cu) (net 11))
 (segment (start 71.28 66.04) (end 80.264 66.04) (width 0.5) (layer B.Cu) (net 11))
 (segment (start 78.74 68.58) (end 73.74 68.58) (width 0.5) (layer F.Cu) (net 12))
 (segment (start 78.74 68.58) (end 78.74 79.502) (width 0.5) (layer B.Cu) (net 12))
 (segment (start 73.66 89.916) (end 76.2 89.916) (width 0.5) (layer F.Cu) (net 13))
 (segment (start 92.672001 77.507999) (end 93.472 76.708) (width 0.5) (layer F.Cu) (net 13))
 (segment (start 87.63 82.55) (end 92.672001 77.507999) (width 0.5) (layer F.Cu) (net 13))
 (segment (start 83.566 82.55) (end 87.63 82.55) (width 0.5) (layer F.Cu) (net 13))
 (segment (start 76.2 89.916) (end 83.566 82.55) (width 0.5) (layer F.Cu) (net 13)))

